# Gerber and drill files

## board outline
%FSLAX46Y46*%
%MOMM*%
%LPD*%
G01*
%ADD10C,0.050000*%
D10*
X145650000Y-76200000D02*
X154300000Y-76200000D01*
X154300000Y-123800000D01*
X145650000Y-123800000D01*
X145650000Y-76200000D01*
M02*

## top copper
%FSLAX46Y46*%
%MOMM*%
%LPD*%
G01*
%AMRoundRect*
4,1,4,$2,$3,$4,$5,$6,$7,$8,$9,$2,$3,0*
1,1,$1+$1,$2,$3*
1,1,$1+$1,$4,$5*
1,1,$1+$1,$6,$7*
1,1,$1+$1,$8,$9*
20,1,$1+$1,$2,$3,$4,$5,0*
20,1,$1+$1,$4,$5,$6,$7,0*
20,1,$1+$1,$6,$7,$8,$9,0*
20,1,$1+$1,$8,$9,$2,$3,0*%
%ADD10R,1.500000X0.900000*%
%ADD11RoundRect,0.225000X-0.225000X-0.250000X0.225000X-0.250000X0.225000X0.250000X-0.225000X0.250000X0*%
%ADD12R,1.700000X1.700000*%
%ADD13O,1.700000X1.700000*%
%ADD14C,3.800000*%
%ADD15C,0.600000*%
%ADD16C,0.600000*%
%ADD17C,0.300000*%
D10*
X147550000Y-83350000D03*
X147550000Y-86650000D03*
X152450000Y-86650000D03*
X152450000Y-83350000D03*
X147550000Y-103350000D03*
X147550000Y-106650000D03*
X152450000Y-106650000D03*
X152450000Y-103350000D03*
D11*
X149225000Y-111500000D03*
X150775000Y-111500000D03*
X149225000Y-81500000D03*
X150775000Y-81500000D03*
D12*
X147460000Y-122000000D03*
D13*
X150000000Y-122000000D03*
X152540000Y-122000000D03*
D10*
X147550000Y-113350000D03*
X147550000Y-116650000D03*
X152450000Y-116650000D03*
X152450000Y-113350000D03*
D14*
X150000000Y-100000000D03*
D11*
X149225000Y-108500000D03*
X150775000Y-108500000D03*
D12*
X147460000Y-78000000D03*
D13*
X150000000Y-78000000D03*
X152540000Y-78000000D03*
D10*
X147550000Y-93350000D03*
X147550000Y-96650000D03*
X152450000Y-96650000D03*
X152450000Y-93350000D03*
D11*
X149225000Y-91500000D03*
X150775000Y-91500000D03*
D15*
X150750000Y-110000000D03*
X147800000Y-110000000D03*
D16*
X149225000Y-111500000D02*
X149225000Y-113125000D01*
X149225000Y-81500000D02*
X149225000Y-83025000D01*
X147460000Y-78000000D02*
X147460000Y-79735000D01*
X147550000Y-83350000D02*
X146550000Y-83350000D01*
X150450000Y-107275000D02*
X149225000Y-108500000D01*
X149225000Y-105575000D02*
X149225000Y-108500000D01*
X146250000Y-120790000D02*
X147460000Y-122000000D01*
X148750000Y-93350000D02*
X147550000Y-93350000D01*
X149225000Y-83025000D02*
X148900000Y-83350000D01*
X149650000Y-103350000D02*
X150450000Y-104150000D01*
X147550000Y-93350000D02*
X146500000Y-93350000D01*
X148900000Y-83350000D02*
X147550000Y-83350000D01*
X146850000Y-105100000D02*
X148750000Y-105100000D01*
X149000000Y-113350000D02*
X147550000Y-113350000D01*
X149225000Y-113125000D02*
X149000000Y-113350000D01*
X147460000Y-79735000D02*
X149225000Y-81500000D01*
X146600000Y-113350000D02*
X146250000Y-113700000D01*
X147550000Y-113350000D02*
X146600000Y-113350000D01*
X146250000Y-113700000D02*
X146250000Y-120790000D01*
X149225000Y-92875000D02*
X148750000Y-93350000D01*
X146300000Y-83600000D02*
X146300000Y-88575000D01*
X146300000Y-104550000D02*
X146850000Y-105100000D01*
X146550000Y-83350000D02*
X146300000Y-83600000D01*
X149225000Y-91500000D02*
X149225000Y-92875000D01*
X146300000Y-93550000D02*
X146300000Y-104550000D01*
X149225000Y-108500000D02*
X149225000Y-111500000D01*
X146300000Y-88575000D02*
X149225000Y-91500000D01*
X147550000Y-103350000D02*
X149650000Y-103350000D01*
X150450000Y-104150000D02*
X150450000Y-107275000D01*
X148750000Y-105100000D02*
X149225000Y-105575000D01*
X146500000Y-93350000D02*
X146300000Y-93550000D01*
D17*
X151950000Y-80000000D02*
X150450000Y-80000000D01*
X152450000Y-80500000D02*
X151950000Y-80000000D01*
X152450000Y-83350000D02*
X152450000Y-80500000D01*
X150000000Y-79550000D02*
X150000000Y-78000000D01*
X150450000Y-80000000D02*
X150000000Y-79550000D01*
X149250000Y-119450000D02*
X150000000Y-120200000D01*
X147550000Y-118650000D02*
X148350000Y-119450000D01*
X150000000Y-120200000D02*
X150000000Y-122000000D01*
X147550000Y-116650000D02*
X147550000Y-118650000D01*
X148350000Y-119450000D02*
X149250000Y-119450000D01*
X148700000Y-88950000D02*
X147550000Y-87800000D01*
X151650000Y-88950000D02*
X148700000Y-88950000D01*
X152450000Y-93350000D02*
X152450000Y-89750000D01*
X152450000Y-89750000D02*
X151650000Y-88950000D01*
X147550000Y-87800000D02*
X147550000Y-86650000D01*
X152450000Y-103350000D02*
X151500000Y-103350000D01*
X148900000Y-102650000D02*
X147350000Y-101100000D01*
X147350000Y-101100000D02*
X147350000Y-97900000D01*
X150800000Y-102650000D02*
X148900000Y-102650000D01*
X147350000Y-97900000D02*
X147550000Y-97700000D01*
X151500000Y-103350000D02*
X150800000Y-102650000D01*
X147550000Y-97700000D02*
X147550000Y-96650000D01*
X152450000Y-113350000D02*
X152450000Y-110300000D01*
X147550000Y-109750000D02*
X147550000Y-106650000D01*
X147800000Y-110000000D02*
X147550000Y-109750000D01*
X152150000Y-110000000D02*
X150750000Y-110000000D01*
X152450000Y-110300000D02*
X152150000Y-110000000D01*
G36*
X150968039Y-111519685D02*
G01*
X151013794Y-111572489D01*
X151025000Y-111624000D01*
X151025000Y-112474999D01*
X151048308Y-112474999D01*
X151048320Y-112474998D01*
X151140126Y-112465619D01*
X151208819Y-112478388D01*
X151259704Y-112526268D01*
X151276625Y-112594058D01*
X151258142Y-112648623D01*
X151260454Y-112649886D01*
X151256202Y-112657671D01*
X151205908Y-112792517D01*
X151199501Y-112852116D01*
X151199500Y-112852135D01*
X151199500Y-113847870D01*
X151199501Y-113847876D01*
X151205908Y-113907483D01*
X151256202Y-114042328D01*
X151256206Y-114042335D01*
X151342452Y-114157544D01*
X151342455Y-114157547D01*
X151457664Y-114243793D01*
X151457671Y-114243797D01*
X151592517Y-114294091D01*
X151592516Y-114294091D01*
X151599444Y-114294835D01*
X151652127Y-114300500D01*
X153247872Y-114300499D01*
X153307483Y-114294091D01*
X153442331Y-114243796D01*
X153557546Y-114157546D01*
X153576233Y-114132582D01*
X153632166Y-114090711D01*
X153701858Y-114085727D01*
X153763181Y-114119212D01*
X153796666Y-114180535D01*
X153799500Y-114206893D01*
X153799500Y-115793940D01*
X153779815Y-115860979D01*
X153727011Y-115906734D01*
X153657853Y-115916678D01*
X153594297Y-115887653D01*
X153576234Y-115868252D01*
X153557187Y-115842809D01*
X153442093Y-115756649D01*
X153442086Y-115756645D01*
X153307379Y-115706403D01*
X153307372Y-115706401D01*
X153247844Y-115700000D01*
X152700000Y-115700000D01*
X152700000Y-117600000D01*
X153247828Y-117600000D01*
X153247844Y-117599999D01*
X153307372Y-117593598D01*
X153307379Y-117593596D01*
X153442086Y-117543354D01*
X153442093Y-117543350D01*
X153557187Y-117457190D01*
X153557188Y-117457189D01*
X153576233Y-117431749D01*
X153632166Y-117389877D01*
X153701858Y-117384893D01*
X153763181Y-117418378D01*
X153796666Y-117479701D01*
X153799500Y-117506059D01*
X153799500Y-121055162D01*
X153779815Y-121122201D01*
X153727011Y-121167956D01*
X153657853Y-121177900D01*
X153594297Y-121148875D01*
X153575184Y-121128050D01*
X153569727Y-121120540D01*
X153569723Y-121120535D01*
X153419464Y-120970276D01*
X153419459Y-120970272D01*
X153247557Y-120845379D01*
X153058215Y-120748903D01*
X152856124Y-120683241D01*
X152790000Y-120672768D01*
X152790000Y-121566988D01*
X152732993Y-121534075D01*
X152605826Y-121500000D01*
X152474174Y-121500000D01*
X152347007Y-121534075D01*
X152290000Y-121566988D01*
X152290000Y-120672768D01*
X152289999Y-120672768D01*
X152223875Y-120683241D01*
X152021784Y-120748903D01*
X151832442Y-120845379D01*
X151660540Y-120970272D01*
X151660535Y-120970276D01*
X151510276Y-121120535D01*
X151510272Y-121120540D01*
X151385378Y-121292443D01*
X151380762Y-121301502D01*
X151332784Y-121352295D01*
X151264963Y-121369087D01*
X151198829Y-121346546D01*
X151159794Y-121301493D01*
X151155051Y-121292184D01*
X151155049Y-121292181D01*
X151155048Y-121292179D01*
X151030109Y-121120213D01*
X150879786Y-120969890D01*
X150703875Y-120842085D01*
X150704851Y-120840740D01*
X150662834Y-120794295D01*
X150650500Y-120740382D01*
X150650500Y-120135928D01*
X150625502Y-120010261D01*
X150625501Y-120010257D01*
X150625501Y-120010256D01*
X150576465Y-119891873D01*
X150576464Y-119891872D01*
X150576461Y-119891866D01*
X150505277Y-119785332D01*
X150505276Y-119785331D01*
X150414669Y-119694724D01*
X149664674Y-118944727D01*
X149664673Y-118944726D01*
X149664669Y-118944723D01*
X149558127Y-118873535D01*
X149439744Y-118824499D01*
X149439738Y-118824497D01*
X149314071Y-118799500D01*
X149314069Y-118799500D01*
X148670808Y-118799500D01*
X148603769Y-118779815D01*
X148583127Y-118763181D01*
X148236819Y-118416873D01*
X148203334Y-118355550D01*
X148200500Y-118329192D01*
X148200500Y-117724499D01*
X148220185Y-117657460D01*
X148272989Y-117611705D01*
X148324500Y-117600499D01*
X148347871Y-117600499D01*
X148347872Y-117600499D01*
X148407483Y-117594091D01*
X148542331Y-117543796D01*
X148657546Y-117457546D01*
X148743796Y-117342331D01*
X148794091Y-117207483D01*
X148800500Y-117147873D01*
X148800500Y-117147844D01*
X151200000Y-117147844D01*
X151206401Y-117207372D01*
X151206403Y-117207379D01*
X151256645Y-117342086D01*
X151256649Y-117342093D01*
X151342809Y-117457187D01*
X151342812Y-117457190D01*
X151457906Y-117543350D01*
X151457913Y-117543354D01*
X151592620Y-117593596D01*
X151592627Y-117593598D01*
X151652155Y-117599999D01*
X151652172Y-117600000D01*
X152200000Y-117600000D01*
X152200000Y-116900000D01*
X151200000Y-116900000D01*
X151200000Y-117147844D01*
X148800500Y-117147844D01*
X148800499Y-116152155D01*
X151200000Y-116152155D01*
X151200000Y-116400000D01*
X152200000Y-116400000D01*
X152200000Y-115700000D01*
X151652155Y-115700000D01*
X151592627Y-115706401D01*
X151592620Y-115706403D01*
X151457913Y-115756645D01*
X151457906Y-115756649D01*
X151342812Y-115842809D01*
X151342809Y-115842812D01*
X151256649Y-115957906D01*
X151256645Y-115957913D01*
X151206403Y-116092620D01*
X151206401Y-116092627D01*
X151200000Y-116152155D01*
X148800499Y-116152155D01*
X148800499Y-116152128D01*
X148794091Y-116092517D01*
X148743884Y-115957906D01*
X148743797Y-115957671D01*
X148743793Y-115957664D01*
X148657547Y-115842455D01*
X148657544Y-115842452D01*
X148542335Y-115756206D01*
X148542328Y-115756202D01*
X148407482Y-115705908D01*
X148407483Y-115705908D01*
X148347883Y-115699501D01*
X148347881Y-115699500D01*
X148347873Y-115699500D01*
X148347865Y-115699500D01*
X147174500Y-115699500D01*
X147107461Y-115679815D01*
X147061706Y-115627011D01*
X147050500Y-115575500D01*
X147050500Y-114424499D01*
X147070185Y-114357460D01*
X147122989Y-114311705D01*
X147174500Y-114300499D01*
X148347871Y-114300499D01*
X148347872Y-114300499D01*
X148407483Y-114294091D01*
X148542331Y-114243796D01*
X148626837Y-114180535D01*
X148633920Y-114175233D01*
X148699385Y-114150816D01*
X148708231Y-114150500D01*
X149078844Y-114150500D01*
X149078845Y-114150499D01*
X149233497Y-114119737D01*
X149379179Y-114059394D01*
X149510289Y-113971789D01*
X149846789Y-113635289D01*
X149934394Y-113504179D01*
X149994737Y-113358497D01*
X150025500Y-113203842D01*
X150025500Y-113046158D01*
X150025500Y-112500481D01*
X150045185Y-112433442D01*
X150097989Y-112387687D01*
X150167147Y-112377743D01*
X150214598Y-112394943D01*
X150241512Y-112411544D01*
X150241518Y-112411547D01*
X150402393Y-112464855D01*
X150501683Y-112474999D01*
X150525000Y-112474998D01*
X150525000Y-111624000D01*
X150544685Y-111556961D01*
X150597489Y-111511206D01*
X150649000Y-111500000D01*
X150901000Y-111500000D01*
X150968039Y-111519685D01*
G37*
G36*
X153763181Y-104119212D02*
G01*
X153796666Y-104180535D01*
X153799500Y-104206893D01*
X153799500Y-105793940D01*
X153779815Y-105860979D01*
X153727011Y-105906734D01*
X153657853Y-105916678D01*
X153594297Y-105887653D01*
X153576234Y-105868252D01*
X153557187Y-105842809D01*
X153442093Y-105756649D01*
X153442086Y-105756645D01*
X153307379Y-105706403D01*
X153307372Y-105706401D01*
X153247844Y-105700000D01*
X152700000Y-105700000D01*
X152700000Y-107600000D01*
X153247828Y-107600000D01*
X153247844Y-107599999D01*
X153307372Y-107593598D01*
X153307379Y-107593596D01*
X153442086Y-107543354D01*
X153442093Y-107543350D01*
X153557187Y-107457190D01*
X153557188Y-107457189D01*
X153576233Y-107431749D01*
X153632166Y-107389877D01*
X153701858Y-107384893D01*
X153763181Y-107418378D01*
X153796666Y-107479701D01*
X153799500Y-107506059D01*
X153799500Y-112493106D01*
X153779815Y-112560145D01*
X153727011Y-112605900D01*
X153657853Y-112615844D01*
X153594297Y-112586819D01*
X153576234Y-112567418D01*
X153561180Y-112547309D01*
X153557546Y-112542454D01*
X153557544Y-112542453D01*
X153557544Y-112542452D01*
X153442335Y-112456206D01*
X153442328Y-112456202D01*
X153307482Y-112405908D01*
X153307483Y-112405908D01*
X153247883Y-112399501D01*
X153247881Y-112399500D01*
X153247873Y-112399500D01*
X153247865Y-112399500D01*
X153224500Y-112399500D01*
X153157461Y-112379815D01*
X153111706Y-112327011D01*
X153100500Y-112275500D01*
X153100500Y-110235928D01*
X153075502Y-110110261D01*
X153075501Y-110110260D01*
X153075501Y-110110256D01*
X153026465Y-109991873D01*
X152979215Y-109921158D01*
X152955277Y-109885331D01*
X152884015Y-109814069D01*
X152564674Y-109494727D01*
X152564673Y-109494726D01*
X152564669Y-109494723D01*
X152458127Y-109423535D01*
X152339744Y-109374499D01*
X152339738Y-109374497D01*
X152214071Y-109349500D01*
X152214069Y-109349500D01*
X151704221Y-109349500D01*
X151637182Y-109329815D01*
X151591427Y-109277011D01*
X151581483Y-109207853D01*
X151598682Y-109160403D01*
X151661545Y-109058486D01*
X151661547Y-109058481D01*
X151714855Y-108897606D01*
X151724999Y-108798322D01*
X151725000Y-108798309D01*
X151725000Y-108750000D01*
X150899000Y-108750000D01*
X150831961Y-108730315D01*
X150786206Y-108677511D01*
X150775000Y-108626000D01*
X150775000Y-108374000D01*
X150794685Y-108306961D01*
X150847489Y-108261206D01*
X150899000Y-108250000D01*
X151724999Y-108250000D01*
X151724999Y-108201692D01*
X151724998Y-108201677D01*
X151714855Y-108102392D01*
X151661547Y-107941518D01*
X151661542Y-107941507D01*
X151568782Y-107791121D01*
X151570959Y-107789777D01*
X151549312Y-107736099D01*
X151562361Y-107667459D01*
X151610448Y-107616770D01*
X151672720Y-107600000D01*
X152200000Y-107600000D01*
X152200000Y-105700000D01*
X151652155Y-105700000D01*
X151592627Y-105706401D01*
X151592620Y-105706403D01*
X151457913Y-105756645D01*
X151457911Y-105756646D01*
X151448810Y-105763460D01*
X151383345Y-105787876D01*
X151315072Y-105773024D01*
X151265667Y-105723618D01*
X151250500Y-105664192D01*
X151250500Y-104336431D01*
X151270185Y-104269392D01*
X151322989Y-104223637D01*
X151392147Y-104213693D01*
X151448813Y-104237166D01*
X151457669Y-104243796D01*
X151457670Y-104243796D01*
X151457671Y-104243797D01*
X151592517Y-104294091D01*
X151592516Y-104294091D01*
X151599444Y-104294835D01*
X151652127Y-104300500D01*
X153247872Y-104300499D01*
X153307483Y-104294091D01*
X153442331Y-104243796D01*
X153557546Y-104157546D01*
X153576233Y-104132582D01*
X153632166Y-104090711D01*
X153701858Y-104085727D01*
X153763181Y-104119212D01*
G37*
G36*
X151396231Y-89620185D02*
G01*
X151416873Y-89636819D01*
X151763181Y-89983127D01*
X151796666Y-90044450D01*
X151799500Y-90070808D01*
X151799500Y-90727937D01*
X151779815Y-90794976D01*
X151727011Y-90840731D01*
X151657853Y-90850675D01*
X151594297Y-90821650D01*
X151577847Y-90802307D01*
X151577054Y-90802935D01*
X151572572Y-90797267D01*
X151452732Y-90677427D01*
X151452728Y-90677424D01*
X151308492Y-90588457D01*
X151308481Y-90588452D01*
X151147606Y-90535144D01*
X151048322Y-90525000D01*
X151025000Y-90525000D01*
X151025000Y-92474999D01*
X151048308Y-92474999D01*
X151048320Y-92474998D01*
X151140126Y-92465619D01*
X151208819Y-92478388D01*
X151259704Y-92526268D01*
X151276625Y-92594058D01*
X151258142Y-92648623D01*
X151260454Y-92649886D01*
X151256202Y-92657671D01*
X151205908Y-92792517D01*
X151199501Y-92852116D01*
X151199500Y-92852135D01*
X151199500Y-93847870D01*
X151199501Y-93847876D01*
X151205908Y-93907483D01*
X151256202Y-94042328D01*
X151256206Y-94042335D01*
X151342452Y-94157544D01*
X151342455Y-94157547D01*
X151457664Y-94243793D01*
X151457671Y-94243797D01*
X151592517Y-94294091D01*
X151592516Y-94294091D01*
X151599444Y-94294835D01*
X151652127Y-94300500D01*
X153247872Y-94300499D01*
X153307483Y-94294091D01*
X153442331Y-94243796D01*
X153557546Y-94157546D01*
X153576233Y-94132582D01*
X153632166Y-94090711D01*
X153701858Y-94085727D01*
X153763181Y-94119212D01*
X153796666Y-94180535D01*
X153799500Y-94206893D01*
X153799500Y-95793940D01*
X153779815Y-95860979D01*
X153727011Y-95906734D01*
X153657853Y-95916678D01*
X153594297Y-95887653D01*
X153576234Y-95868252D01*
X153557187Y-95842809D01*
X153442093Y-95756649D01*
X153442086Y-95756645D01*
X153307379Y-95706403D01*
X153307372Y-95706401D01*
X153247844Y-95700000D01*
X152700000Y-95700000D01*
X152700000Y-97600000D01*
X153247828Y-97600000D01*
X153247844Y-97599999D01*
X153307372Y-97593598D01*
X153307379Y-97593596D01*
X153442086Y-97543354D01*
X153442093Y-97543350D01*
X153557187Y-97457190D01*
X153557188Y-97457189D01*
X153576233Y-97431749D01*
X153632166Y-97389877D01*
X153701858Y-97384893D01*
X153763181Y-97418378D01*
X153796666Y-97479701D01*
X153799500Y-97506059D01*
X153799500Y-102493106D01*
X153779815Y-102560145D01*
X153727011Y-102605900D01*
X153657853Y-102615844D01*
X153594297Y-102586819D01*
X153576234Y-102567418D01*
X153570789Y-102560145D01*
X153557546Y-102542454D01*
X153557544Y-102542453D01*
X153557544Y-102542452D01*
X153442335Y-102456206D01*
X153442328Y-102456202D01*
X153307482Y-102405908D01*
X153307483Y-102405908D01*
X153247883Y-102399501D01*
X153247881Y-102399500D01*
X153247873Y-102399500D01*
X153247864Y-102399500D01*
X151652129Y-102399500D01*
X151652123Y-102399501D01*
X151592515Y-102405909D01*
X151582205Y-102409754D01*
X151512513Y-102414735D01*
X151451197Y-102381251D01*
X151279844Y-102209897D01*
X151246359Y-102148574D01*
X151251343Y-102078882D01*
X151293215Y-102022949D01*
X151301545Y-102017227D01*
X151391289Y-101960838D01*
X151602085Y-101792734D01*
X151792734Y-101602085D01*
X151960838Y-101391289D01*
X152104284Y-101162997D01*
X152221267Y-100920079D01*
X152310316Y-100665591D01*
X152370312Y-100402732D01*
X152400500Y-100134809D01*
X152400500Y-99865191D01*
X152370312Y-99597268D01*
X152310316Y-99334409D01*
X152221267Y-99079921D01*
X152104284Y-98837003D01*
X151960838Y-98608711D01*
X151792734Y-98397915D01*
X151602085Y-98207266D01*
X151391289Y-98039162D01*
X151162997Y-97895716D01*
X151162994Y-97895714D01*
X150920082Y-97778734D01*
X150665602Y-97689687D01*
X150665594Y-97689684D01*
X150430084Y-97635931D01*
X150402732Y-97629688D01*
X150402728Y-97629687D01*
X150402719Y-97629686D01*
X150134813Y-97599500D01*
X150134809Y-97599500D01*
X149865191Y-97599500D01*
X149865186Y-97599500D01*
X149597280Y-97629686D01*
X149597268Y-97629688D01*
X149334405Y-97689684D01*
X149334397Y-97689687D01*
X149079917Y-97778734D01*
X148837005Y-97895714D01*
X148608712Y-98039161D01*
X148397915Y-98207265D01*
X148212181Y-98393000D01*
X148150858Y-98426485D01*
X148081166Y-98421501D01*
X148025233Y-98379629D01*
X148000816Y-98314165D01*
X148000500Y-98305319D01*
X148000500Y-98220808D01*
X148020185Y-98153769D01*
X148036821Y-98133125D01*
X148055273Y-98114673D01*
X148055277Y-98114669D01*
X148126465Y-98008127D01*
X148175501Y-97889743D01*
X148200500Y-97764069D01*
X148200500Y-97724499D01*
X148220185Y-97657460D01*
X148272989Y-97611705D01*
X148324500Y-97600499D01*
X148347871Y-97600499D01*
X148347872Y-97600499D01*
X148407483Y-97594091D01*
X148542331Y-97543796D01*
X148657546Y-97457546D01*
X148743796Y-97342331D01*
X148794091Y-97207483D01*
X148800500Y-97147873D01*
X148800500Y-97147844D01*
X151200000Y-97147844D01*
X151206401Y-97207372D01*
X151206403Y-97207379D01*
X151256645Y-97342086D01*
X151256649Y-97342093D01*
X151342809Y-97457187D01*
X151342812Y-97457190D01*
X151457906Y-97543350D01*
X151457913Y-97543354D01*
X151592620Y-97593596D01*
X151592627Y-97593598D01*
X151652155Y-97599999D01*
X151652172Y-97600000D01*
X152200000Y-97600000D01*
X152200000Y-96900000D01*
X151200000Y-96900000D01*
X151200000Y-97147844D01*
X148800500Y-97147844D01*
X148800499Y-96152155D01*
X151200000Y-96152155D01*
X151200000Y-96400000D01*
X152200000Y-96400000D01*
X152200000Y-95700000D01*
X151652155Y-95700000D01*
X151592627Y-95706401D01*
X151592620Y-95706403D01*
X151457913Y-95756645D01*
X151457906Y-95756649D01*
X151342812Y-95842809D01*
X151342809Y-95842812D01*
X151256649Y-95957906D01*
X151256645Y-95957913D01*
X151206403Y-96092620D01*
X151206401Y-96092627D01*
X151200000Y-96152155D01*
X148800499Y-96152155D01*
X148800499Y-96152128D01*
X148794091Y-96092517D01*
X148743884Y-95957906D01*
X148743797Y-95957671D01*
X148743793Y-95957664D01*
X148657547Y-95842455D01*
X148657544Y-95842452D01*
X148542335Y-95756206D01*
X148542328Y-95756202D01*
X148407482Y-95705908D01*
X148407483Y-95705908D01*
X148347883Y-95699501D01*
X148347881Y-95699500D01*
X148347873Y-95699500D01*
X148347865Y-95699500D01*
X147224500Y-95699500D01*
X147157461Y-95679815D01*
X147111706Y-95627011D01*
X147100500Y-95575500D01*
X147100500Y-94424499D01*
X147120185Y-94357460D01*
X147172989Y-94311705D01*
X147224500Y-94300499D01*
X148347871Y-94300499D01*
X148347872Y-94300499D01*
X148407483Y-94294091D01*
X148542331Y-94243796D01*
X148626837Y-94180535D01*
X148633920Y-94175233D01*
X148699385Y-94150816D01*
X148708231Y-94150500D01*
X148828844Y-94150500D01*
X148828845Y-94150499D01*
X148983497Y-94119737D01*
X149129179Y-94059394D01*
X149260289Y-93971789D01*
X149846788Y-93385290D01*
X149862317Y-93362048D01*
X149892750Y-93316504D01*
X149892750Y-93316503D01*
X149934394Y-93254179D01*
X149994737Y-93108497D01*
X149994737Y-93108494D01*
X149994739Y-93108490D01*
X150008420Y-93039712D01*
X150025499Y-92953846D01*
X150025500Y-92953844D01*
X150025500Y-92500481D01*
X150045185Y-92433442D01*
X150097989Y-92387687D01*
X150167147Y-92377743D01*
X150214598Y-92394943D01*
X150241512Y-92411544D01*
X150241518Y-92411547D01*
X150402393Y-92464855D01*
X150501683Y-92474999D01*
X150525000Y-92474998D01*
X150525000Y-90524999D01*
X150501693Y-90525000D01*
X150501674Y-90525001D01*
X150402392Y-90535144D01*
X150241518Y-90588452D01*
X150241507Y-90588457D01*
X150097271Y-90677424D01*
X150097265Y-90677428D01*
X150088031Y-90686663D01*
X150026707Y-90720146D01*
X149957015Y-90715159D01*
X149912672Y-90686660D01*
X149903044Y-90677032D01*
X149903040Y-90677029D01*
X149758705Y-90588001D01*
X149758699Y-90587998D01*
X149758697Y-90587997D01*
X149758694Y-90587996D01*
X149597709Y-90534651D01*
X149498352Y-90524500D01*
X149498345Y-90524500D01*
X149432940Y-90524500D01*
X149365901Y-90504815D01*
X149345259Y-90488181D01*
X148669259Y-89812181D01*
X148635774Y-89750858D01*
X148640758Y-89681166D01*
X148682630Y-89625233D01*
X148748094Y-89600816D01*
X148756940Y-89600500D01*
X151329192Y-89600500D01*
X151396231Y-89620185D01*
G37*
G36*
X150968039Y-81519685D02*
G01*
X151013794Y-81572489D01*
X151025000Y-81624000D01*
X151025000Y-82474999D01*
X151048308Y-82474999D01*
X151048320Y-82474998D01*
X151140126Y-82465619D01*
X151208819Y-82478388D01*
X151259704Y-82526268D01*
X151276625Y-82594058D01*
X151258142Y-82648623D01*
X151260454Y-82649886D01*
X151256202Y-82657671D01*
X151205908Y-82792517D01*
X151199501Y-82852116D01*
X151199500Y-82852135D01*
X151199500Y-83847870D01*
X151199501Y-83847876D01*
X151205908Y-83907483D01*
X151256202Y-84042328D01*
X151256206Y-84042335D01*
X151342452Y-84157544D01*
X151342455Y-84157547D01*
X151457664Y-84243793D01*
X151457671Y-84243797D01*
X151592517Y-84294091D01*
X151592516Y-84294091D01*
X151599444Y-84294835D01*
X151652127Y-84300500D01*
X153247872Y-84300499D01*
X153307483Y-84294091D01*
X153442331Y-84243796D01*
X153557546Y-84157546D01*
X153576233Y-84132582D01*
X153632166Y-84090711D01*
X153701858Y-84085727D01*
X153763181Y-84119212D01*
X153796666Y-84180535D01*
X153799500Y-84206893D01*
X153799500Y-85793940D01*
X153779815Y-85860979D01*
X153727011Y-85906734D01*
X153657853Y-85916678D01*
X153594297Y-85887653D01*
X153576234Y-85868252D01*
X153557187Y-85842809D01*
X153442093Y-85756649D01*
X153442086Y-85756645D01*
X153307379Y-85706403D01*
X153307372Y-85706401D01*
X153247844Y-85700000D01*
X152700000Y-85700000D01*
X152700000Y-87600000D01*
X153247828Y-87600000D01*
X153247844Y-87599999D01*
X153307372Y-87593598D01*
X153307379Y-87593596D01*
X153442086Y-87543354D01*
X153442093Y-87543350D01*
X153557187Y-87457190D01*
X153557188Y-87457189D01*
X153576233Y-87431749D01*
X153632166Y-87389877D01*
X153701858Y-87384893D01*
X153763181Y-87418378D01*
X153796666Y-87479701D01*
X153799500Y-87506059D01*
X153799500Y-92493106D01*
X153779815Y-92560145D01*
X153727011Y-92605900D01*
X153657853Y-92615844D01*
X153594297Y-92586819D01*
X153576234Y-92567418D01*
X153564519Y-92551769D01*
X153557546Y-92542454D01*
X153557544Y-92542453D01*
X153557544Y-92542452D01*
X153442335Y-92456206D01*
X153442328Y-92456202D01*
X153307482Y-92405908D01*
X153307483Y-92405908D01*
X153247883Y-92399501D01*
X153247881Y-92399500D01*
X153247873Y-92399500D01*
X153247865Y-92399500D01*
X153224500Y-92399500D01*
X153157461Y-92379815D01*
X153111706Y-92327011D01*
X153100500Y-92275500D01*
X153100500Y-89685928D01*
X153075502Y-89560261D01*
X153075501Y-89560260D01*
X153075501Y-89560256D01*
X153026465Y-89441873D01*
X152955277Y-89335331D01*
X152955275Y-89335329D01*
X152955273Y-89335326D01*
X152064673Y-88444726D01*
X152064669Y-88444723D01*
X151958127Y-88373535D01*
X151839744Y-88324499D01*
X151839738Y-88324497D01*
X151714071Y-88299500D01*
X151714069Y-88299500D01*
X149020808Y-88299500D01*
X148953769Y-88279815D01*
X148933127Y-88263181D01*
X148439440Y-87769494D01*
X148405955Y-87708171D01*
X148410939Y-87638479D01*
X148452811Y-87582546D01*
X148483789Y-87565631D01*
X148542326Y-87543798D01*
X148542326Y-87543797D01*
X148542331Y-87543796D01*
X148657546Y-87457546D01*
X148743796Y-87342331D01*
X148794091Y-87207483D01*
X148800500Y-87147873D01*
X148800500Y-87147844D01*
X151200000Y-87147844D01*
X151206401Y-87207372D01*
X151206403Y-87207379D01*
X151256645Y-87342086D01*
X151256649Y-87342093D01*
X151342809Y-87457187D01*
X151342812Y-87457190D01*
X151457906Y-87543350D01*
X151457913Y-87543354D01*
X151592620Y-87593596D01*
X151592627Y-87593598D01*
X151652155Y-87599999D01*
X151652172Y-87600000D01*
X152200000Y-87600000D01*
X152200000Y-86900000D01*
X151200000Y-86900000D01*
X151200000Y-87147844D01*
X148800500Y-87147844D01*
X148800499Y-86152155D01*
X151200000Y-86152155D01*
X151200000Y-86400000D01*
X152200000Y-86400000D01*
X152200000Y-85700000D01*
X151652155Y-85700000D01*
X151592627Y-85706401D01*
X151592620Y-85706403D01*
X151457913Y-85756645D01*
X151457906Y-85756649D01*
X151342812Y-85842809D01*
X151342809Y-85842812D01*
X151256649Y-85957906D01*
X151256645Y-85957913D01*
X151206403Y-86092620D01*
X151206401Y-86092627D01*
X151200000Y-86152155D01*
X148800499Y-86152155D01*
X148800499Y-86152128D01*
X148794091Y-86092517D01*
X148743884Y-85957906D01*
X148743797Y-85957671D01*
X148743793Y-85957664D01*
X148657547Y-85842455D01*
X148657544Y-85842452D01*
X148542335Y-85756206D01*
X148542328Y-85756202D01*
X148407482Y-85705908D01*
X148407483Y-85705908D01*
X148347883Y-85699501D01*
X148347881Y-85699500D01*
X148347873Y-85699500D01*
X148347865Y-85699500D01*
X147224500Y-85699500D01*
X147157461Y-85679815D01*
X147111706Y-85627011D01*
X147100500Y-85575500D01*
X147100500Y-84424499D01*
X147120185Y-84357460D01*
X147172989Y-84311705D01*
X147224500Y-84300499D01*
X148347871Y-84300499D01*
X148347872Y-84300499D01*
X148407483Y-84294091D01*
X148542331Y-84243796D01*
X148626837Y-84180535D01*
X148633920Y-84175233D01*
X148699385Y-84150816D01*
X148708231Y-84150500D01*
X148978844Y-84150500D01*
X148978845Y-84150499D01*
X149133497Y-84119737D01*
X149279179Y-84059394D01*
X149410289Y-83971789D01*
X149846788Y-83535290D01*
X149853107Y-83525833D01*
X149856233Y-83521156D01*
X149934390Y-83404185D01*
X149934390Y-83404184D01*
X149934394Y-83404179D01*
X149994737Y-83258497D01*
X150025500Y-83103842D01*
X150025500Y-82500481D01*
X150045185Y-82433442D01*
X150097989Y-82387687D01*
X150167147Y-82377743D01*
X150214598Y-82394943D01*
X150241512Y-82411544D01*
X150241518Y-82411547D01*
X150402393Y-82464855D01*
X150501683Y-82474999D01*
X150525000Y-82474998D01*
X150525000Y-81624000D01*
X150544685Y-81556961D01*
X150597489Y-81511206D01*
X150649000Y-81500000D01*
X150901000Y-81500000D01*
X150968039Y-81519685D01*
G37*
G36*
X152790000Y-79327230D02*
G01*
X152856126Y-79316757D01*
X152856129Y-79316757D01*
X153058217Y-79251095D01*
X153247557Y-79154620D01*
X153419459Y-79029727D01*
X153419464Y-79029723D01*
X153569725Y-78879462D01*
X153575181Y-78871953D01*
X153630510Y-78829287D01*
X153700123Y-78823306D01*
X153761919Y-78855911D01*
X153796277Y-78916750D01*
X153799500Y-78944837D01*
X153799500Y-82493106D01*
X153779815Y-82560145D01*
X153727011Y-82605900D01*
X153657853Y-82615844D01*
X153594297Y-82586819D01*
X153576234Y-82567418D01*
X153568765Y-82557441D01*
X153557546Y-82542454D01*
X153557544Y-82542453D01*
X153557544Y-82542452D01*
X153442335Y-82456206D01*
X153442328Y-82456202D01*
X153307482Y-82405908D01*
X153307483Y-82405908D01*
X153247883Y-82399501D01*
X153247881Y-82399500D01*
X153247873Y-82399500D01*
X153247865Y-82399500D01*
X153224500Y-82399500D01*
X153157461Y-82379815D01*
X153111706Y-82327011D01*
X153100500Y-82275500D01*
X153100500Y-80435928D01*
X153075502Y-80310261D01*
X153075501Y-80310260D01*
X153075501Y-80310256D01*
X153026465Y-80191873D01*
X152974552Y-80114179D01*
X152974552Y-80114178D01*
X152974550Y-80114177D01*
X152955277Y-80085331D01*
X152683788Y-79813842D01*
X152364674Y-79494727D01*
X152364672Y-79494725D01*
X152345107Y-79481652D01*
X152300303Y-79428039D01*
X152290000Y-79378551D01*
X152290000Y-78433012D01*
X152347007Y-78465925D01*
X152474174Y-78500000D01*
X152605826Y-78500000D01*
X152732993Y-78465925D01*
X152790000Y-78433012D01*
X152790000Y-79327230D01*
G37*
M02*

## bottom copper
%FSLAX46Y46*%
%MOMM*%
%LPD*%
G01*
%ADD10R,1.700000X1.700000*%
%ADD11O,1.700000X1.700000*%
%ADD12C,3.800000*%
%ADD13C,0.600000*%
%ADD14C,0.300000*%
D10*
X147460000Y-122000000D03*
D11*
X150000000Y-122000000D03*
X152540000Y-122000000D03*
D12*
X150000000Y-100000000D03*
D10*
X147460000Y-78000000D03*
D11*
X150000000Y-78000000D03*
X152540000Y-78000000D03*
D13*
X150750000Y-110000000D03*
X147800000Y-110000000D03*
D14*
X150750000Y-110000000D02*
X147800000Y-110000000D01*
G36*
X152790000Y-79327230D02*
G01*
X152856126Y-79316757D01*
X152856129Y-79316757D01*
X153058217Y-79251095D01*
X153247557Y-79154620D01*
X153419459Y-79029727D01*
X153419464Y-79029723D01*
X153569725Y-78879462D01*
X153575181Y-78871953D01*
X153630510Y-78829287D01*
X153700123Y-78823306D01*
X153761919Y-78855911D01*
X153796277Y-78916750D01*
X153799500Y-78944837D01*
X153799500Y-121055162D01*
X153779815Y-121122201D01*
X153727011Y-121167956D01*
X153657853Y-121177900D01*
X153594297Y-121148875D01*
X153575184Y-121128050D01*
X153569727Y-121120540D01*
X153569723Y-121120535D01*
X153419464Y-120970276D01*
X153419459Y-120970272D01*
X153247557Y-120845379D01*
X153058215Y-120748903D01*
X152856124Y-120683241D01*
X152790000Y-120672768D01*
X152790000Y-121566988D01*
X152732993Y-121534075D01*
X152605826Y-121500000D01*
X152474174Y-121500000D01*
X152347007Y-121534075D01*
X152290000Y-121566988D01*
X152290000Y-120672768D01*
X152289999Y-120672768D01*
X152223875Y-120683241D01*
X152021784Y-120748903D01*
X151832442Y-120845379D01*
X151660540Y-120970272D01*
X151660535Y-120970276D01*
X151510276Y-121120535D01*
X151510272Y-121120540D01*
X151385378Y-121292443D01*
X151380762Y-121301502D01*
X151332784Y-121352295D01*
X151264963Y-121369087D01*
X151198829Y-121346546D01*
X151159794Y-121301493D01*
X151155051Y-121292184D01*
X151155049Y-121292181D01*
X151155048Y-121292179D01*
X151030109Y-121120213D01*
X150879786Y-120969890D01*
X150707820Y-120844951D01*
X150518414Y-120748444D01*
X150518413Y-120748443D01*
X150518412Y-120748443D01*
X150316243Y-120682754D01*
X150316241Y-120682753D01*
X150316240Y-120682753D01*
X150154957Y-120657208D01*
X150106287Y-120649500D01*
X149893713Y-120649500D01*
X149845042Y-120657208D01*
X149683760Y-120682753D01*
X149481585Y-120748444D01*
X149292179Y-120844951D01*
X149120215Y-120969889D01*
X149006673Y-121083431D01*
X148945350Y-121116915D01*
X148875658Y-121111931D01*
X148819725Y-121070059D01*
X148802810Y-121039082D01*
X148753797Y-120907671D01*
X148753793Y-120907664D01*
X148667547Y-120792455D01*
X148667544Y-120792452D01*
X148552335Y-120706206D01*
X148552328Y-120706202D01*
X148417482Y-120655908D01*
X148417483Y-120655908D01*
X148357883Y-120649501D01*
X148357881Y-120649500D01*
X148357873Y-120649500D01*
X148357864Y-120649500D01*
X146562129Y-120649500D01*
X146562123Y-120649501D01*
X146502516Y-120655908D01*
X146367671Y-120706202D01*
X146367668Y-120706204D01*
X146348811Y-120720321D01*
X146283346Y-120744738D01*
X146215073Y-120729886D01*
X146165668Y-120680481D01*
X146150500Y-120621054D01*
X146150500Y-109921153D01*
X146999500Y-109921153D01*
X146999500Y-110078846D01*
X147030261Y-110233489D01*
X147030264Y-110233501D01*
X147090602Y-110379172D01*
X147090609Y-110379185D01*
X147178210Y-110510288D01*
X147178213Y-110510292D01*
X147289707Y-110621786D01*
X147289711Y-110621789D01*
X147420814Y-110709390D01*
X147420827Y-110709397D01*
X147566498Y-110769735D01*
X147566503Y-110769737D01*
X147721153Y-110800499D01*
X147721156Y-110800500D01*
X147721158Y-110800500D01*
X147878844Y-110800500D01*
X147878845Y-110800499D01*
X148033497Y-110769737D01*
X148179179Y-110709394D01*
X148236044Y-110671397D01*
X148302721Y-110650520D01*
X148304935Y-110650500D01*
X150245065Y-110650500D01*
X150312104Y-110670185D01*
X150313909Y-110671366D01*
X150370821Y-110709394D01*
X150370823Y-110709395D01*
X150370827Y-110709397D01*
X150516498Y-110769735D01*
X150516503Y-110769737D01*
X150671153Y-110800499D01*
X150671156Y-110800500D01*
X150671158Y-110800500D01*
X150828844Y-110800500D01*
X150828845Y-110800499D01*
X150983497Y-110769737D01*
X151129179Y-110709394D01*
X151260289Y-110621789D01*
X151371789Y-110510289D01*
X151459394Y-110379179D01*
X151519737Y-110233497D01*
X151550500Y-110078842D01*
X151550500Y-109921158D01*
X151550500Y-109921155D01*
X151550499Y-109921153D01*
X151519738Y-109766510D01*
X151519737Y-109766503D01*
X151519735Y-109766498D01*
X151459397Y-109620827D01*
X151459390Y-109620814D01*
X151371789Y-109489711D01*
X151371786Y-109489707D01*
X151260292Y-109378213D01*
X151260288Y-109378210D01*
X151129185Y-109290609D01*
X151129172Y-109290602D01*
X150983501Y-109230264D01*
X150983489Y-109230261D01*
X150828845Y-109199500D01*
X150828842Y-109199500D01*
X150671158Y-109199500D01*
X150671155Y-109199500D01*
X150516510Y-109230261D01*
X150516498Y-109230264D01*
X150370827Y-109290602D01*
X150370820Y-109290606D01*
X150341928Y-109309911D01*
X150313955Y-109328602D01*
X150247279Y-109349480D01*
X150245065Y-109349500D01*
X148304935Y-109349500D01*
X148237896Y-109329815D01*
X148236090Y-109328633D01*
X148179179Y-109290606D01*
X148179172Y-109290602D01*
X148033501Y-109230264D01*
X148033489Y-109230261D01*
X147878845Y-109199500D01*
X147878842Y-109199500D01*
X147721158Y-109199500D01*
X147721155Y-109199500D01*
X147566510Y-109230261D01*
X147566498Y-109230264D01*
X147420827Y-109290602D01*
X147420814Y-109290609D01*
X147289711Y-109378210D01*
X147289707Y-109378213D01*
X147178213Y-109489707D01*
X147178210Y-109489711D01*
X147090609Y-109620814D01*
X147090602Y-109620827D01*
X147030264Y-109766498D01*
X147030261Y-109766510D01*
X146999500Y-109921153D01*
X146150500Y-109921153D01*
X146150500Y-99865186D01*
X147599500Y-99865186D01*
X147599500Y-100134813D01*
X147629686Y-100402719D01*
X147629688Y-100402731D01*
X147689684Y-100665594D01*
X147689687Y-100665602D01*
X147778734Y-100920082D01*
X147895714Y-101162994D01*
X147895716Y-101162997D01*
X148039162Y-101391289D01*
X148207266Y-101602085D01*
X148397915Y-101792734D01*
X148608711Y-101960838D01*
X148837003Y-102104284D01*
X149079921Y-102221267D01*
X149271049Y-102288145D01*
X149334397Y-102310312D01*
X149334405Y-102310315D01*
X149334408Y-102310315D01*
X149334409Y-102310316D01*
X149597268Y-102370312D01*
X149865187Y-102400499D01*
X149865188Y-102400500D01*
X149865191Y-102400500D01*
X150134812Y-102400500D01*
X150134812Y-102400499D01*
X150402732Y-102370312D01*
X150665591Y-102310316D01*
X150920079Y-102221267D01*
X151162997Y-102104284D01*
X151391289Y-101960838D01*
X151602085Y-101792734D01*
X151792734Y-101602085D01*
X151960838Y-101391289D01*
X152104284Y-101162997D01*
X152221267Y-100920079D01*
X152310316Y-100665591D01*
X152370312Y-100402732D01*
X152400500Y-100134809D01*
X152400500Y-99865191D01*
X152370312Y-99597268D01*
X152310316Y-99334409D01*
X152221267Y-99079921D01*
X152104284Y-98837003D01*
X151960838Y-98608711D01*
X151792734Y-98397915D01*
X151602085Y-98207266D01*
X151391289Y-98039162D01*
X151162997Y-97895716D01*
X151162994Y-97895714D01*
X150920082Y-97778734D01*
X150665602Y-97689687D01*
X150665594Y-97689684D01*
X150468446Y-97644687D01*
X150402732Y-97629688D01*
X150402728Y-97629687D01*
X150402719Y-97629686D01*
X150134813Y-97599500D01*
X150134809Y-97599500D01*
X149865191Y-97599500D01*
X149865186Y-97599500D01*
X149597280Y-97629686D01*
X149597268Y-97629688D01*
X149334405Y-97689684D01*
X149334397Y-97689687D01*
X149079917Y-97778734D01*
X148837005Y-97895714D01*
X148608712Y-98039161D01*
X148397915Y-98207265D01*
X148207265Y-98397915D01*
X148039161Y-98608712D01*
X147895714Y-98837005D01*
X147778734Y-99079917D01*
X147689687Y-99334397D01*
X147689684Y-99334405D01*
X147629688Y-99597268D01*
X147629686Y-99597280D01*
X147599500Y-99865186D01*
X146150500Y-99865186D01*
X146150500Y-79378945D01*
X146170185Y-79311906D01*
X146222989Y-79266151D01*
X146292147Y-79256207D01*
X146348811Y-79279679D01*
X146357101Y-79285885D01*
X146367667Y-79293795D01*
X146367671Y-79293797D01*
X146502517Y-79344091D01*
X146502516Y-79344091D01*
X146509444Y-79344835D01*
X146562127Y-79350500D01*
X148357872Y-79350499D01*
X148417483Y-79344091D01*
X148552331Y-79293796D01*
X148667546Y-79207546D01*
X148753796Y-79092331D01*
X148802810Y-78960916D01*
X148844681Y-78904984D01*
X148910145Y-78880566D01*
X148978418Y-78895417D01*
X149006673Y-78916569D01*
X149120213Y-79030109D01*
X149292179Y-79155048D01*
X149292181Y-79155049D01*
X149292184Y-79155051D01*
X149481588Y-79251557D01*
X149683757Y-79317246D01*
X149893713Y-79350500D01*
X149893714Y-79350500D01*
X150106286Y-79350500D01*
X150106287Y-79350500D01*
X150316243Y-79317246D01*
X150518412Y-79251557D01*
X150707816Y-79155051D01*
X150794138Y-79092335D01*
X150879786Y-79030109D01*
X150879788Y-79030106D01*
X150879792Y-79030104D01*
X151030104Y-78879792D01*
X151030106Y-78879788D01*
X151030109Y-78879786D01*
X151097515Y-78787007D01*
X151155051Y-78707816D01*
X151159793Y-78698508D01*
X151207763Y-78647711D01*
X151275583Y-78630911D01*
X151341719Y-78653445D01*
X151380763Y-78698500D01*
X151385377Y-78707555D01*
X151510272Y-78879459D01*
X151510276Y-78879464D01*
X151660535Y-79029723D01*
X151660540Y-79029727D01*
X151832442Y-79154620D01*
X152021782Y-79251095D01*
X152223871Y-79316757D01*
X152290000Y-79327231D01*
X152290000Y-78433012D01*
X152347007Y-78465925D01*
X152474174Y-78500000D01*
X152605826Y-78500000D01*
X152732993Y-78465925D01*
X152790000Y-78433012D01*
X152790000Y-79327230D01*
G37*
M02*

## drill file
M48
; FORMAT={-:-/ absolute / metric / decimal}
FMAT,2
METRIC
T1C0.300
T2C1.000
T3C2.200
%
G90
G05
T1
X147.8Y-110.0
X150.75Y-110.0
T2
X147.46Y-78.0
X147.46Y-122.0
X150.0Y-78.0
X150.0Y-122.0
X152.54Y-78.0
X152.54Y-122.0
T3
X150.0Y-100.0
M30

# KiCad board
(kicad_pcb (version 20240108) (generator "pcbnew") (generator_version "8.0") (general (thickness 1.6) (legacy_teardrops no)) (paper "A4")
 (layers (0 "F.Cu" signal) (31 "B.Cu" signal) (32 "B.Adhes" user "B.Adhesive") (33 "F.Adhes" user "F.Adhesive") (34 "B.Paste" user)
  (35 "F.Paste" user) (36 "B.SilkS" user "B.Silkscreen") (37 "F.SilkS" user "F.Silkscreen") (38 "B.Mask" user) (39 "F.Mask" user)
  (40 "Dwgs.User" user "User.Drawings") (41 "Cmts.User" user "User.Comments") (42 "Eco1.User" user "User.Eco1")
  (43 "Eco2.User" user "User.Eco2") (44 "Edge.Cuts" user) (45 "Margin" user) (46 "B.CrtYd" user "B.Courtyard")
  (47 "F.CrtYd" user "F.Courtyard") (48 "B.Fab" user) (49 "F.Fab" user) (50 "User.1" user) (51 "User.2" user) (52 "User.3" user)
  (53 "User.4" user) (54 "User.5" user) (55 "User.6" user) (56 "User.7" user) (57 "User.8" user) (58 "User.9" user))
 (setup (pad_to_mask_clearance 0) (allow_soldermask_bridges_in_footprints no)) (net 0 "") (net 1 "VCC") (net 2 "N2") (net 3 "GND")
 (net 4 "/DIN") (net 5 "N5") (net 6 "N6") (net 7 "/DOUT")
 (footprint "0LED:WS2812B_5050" (layer "F.Cu") (at 150 85 180)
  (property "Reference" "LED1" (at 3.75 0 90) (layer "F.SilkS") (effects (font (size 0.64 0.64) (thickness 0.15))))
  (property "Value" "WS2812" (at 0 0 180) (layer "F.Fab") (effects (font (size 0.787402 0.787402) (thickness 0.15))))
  (pad "1-VDD" smd rect (at 2.45 1.65 180) (size 1.5 0.9) (layers "F.Cu" "F.Paste" "F.Mask") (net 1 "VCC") (solder_mask_margin 0.102))
  (pad "2-DOUT" smd rect (at 2.45 -1.65 180) (size 1.5 0.9) (layers "F.Cu" "F.Paste" "F.Mask") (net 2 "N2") (solder_mask_margin 0.102))
  (pad "3-GND" smd rect (at -2.45 -1.65 180) (size 1.5 0.9) (layers "F.Cu" "F.Paste" "F.Mask") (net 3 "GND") (solder_mask_margin 0.102))
  (pad "4-DIN" smd rect (at -2.45 1.65 180) (size 1.5 0.9) (layers "F.Cu" "F.Paste" "F.Mask") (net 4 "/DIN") (solder_mask_margin 0.102)))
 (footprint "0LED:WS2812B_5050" (layer "F.Cu") (at 150 105 180)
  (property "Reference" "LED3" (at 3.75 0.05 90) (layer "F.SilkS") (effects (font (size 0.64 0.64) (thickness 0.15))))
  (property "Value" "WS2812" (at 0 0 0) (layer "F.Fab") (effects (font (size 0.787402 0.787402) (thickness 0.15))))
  (pad "1-VDD" smd rect (at 2.45 1.65 180) (size 1.5 0.9) (layers "F.Cu" "F.Paste" "F.Mask") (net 1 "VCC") (solder_mask_margin 0.102))
  (pad "2-DOUT" smd rect (at 2.45 -1.65 180) (size 1.5 0.9) (layers "F.Cu" "F.Paste" "F.Mask") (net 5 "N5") (solder_mask_margin 0.102))
  (pad "3-GND" smd rect (at -2.45 -1.65 180) (size 1.5 0.9) (layers "F.Cu" "F.Paste" "F.Mask") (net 3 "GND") (solder_mask_margin 0.102))
  (pad "4-DIN" smd rect (at -2.45 1.65 180) (size 1.5 0.9) (layers "F.Cu" "F.Paste" "F.Mask") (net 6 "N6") (solder_mask_margin 0.102)))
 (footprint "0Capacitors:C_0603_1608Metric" (layer "F.Cu") (at 150 111.5)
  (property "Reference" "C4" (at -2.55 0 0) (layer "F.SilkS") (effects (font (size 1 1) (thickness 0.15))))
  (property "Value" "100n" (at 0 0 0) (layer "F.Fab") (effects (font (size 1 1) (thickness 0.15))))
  (pad "1" smd roundrect (at -0.775 0) (size 0.9 0.95) (layers "F.Cu" "F.Paste" "F.Mask") (roundrect_rratio 0.25) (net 1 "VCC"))
  (pad "2" smd roundrect (at 0.775 0) (size 0.9 0.95) (layers "F.Cu" "F.Paste" "F.Mask") (roundrect_rratio 0.25) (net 3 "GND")))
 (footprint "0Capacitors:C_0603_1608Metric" (layer "F.Cu") (at 150 81.5)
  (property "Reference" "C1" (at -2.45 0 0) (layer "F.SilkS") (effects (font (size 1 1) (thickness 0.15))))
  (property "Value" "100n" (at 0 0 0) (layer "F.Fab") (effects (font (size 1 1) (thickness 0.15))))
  (pad "1" smd roundrect (at -0.775 0) (size 0.9 0.95) (layers "F.Cu" "F.Paste" "F.Mask") (roundrect_rratio 0.25) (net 1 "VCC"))
  (pad "2" smd roundrect (at 0.775 0) (size 0.9 0.95) (layers "F.Cu" "F.Paste" "F.Mask") (roundrect_rratio 0.25) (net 3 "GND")))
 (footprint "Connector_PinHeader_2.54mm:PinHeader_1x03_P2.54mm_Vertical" (layer "F.Cu") (at 147.46 122 90)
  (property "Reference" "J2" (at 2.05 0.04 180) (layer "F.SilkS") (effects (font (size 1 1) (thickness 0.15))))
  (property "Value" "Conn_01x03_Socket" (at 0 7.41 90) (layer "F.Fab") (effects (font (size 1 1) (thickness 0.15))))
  (pad "1" thru_hole rect (at 0 0 90) (size 1.7 1.7) (drill 1) (layers "*.Cu" "*.Mask") (remove_unused_layers no) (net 1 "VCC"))
  (pad "2" thru_hole oval (at 0 2.54 90) (size 1.7 1.7) (drill 1) (layers "*.Cu" "*.Mask") (remove_unused_layers no) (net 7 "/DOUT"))
  (pad "3" thru_hole oval (at 0 5.08 90) (size 1.7 1.7) (drill 1) (layers "*.Cu" "*.Mask") (remove_unused_layers no) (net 3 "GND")))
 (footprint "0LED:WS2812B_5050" (layer "F.Cu") (at 150 115 180)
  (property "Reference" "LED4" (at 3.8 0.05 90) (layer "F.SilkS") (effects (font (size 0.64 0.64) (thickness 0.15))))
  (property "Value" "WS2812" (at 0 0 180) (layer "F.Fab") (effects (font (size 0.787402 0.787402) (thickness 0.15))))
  (pad "1-VDD" smd rect (at 2.45 1.65 180) (size 1.5 0.9) (layers "F.Cu" "F.Paste" "F.Mask") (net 1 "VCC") (solder_mask_margin 0.102))
  (pad "2-DOUT" smd rect (at 2.45 -1.65 180) (size 1.5 0.9) (layers "F.Cu" "F.Paste" "F.Mask") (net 7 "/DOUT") (solder_mask_margin 0.102))
  (pad "3-GND" smd rect (at -2.45 -1.65 180) (size 1.5 0.9) (layers "F.Cu" "F.Paste" "F.Mask") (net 3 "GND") (solder_mask_margin 0.102))
  (pad "4-DIN" smd rect (at -2.45 1.65 180) (size 1.5 0.9) (layers "F.Cu" "F.Paste" "F.Mask") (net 5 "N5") (solder_mask_margin 0.102)))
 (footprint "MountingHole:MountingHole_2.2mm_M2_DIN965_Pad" (layer "F.Cu") (at 150 100)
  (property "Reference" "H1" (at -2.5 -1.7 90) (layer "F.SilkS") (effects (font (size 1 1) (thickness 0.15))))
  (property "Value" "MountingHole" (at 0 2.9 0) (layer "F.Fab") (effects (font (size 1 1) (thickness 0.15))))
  (pad "1" thru_hole circle (at 0 0) (size 3.8 3.8) (drill 2.2) (layers "*.Cu" "*.Mask") (remove_unused_layers no)))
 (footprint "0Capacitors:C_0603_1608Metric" (layer "F.Cu") (at 150 108.5)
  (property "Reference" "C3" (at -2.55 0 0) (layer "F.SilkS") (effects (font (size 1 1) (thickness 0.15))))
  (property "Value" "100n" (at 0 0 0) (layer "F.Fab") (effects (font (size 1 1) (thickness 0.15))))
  (pad "1" smd roundrect (at -0.775 0) (size 0.9 0.95) (layers "F.Cu" "F.Paste" "F.Mask") (roundrect_rratio 0.25) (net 1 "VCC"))
  (pad "2" smd roundrect (at 0.775 0) (size 0.9 0.95) (layers "F.Cu" "F.Paste" "F.Mask") (roundrect_rratio 0.25) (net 3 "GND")))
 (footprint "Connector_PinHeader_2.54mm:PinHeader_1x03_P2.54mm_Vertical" (layer "F.Cu") (at 147.46 78 90)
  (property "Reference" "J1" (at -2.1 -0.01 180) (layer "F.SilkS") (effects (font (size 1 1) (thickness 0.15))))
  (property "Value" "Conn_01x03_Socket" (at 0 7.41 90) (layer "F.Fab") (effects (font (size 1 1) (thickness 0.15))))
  (pad "1" thru_hole rect (at 0 0 90) (size 1.7 1.7) (drill 1) (layers "*.Cu" "*.Mask") (remove_unused_layers no) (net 1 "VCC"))
  (pad "2" thru_hole oval (at 0 2.54 90) (size 1.7 1.7) (drill 1) (layers "*.Cu" "*.Mask") (remove_unused_layers no) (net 4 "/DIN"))
  (pad "3" thru_hole oval (at 0 5.08 90) (size 1.7 1.7) (drill 1) (layers "*.Cu" "*.Mask") (remove_unused_layers no) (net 3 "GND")))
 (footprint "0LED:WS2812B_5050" (layer "F.Cu") (at 150 95 180)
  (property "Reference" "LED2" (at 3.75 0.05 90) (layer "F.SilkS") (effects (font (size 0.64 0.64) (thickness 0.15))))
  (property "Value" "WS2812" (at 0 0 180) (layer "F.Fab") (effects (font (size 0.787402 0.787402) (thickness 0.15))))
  (pad "1-VDD" smd rect (at 2.45 1.65 180) (size 1.5 0.9) (layers "F.Cu" "F.Paste" "F.Mask") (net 1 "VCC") (solder_mask_margin 0.102))
  (pad "2-DOUT" smd rect (at 2.45 -1.65 180) (size 1.5 0.9) (layers "F.Cu" "F.Paste" "F.Mask") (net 6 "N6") (solder_mask_margin 0.102))
  (pad "3-GND" smd rect (at -2.45 -1.65 180) (size 1.5 0.9) (layers "F.Cu" "F.Paste" "F.Mask") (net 3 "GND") (solder_mask_margin 0.102))
  (pad "4-DIN" smd rect (at -2.45 1.65 180) (size 1.5 0.9) (layers "F.Cu" "F.Paste" "F.Mask") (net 2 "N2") (solder_mask_margin 0.102)))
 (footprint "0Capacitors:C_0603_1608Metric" (layer "F.Cu") (at 150 91.5)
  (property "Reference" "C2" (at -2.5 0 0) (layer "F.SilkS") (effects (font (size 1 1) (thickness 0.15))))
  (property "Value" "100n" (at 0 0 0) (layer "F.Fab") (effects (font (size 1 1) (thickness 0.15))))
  (pad "1" smd roundrect (at -0.775 0) (size 0.9 0.95) (layers "F.Cu" "F.Paste" "F.Mask") (roundrect_rratio 0.25) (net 1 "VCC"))
  (pad "2" smd roundrect (at 0.775 0) (size 0.9 0.95) (layers "F.Cu" "F.Paste" "F.Mask") (roundrect_rratio 0.25) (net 3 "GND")))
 (gr_rect (start 145.65 76.2) (end 154.3 123.8) (stroke (width 0.05) (type default)) (fill none) (layer "Edge.Cuts"))
 (segment (start 149.225 111.5) (end 149.225 113.125) (width 0.6) (layer "F.Cu") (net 1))
 (segment (start 149.225 81.5) (end 149.225 83.025) (width 0.6) (layer "F.Cu") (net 1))
 (segment (start 147.46 78) (end 147.46 79.735) (width 0.6) (layer "F.Cu") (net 1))
 (segment (start 147.55 83.35) (end 146.55 83.35) (width 0.6) (layer "F.Cu") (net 1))
 (segment (start 150.45 107.275) (end 149.225 108.5) (width 0.6) (layer "F.Cu") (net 1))
 (segment (start 149.225 105.575) (end 149.225 108.5) (width 0.6) (layer "F.Cu") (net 1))
 (segment (start 146.25 120.79) (end 147.46 122) (width 0.6) (layer "F.Cu") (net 1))
 (segment (start 148.75 93.35) (end 147.55 93.35) (width 0.6) (layer "F.Cu") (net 1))
 (segment (start 149.225 83.025) (end 148.9 83.35) (width 0.6) (layer "F.Cu") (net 1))
 (segment (start 149.65 103.35) (end 150.45 104.15) (width 0.6) (layer "F.Cu") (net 1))
 (segment (start 147.55 93.35) (end 146.5 93.35) (width 0.6) (layer "F.Cu") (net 1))
 (segment (start 148.9 83.35) (end 147.55 83.35) (width 0.6) (layer "F.Cu") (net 1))
 (segment (start 146.85 105.1) (end 148.75 105.1) (width 0.6) (layer "F.Cu") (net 1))
 (segment (start 149 113.35) (end 147.55 113.35) (width 0.6) (layer "F.Cu") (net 1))
 (segment (start 149.225 113.125) (end 149 113.35) (width 0.6) (layer "F.Cu") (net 1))
 (segment (start 147.46 79.735) (end 149.225 81.5) (width 0.6) (layer "F.Cu") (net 1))
 (segment (start 146.6 113.35) (end 146.25 113.7) (width 0.6) (layer "F.Cu") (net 1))
 (segment (start 147.55 113.35) (end 146.6 113.35) (width 0.6) (layer "F.Cu") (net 1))
 (segment (start 146.25 113.7) (end 146.25 120.79) (width 0.6) (layer "F.Cu") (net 1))
 (segment (start 149.225 92.875) (end 148.75 93.35) (width 0.6) (layer "F.Cu") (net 1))
 (segment (start 146.3 83.6) (end 146.3 88.575) (width 0.6) (layer "F.Cu") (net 1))
 (segment (start 146.3 104.55) (end 146.85 105.1) (width 0.6) (layer "F.Cu") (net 1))
 (segment (start 146.55 83.35) (end 146.3 83.6) (width 0.6) (layer "F.Cu") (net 1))
 (segment (start 149.225 91.5) (end 149.225 92.875) (width 0.6) (layer "F.Cu") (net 1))
 (segment (start 146.3 93.55) (end 146.3 104.55) (width 0.6) (layer "F.Cu") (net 1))
 (segment (start 149.225 108.5) (end 149.225 111.5) (width 0.6) (layer "F.Cu") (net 1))
 (segment (start 146.3 88.575) (end 149.225 91.5) (width 0.6) (layer "F.Cu") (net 1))
 (segment (start 147.55 103.35) (end 149.65 103.35) (width 0.6) (layer "F.Cu") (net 1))
 (segment (start 150.45 104.15) (end 150.45 107.275) (width 0.6) (layer "F.Cu") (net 1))
 (segment (start 148.75 105.1) (end 149.225 105.575) (width 0.6) (layer "F.Cu") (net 1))
 (segment (start 146.5 93.35) (end 146.3 93.55) (width 0.6) (layer "F.Cu") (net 1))
 (segment (start 151.95 80) (end 150.45 80) (width 0.3) (layer "F.Cu") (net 4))
 (segment (start 152.45 80.5) (end 151.95 80) (width 0.3) (layer "F.Cu") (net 4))
 (segment (start 152.45 83.35) (end 152.45 80.5) (width 0.3) (layer "F.Cu") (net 4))
 (segment (start 150 79.55) (end 150 78) (width 0.3) (layer "F.Cu") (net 4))
 (segment (start 150.45 80) (end 150 79.55) (width 0.3) (layer "F.Cu") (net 4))
 (segment (start 149.25 119.45) (end 150 120.2) (width 0.3) (layer "F.Cu") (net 7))
 (segment (start 147.55 118.65) (end 148.35 119.45) (width 0.3) (layer "F.Cu") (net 7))
 (segment (start 150 120.2) (end 150 122) (width 0.3) (layer "F.Cu") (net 7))
 (segment (start 147.55 116.65) (end 147.55 118.65) (width 0.3) (layer "F.Cu") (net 7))
 (segment (start 148.35 119.45) (end 149.25 119.45) (width 0.3) (layer "F.Cu") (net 7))
 (segment (start 148.7 88.95) (end 147.55 87.8) (width 0.3) (layer "F.Cu") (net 2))
 (segment (start 151.65 88.95) (end 148.7 88.95) (width 0.3) (layer "F.Cu") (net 2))
 (segment (start 152.45 93.35) (end 152.45 89.75) (width 0.3) (layer "F.Cu") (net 2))
 (segment (start 152.45 89.75) (end 151.65 88.95) (width 0.3) (layer "F.Cu") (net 2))
 (segment (start 147.55 87.8) (end 147.55 86.65) (width 0.3) (layer "F.Cu") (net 2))
 (segment (start 152.45 103.35) (end 151.5 103.35) (width 0.3) (layer "F.Cu") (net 6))
 (segment (start 148.9 102.65) (end 147.35 101.1) (width 0.3) (layer "F.Cu") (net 6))
 (segment (start 147.35 101.1) (end 147.35 97.9) (width 0.3) (layer "F.Cu") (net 6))
 (segment (start 150.8 102.65) (end 148.9 102.65) (width 0.3) (layer "F.Cu") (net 6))
 (segment (start 147.35 97.9) (end 147.55 97.7) (width 0.3) (layer "F.Cu") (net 6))
 (segment (start 151.5 103.35) (end 150.8 102.65) (width 0.3) (layer "F.Cu") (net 6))
 (segment (start 147.55 97.7) (end 147.55 96.65) (width 0.3) (layer "F.Cu") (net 6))
 (segment (start 152.45 113.35) (end 152.45 110.3) (width 0.3) (layer "F.Cu") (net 5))
 (segment (start 147.55 109.75) (end 147.55 106.65) (width 0.3) (layer "F.Cu") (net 5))
 (segment (start 147.8 110) (end 147.55 109.75) (width 0.3) (layer "F.Cu") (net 5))
 (segment (start 152.15 110) (end 150.75 110) (width 0.3) (layer "F.Cu") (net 5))
 (segment (start 152.45 110.3) (end 152.15 110) (width 0.3) (layer "F.Cu") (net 5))
 (via (at 150.75 110) (size 0.6) (drill 0.3) (layers "F.Cu" "B.Cu") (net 5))
 (via (at 147.8 110) (size 0.6) (drill 0.3) (layers "F.Cu" "B.Cu") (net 5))
 (segment (start 150.75 110) (end 147.8 110) (width 0.3) (layer "B.Cu") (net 5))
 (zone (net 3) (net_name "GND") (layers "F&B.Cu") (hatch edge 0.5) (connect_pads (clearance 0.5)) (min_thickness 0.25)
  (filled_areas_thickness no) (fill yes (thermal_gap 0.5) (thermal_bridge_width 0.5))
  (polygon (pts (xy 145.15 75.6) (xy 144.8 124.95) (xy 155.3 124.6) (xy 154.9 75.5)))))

